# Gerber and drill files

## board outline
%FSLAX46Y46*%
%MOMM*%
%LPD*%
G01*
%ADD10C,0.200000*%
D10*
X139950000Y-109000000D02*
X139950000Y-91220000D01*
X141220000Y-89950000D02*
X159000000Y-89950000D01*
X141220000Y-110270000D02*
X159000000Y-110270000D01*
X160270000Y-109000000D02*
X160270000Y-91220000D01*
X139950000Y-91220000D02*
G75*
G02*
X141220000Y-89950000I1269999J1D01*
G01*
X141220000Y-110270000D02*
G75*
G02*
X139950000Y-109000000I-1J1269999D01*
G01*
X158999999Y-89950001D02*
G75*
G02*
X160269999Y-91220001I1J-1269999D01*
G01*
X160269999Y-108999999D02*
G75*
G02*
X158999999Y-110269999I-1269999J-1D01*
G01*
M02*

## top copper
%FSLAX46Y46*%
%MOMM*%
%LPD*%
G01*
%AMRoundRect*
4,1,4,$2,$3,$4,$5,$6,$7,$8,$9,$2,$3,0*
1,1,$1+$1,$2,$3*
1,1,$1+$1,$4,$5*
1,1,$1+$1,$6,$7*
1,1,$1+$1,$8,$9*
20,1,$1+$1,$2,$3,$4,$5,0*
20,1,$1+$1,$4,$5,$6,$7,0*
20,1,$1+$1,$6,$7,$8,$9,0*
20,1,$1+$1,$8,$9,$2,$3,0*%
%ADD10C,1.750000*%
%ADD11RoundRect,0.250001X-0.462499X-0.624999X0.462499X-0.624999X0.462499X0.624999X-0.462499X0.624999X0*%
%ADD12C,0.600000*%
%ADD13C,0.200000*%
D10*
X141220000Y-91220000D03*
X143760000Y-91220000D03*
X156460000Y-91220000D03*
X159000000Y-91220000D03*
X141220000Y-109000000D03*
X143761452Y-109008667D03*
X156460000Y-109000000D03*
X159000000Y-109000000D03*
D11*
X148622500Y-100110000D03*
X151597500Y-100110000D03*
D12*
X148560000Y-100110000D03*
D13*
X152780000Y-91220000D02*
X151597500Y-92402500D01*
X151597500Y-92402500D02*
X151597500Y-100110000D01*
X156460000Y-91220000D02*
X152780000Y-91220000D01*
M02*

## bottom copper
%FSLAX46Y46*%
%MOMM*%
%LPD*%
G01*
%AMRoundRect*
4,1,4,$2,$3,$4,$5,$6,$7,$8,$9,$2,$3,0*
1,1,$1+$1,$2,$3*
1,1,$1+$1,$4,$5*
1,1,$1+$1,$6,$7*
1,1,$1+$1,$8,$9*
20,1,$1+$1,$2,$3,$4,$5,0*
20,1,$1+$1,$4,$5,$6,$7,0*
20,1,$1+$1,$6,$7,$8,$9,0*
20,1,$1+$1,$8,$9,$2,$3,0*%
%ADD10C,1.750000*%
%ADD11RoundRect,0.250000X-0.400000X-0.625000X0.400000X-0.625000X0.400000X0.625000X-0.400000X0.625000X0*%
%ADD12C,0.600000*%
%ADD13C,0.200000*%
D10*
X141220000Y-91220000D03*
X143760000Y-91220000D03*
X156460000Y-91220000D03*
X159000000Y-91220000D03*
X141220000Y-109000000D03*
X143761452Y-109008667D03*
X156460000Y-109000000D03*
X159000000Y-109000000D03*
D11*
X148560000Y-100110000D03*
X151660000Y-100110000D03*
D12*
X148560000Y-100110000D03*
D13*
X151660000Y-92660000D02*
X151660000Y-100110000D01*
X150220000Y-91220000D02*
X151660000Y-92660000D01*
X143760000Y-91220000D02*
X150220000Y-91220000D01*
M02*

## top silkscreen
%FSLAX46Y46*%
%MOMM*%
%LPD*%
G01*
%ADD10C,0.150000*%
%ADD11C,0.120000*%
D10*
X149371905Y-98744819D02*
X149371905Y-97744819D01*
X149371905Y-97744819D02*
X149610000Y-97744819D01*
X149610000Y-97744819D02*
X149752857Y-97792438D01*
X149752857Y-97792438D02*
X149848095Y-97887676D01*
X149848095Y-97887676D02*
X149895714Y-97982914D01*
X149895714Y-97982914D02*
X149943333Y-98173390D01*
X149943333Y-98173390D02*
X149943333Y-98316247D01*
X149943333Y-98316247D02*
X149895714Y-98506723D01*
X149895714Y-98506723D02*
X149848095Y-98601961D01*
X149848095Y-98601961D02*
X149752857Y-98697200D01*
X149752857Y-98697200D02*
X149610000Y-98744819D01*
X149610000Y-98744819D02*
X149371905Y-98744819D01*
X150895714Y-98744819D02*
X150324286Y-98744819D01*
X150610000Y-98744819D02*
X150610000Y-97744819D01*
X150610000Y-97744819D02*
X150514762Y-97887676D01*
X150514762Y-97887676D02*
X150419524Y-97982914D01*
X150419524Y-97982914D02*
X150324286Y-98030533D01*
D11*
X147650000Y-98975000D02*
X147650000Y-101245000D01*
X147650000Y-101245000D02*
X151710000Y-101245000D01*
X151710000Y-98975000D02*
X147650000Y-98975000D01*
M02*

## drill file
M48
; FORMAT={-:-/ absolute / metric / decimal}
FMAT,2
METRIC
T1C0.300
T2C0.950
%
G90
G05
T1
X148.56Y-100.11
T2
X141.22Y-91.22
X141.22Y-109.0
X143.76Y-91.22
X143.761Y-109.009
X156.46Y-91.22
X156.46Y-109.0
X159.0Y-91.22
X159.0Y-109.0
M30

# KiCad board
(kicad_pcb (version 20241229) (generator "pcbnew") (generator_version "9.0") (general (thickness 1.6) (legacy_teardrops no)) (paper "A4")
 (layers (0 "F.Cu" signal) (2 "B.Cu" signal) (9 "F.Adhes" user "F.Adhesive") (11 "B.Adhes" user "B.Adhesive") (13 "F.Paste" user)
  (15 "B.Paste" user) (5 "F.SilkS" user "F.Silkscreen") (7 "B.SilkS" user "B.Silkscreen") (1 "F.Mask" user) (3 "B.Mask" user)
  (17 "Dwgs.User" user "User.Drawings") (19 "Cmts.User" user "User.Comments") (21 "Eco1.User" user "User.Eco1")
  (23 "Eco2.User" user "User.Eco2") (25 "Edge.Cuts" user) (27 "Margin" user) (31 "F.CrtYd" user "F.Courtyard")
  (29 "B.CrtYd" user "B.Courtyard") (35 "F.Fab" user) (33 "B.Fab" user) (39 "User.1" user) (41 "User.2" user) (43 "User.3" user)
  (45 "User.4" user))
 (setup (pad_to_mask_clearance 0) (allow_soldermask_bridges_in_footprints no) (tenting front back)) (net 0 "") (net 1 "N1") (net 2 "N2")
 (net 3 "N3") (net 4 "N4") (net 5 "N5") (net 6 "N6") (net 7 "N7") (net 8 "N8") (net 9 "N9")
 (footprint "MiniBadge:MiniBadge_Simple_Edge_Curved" (layer "F.Cu") (at 150.11 100.11)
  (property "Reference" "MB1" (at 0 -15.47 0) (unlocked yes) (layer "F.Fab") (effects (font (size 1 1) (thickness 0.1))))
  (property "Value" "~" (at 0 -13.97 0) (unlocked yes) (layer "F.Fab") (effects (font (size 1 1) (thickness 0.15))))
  (fp_line (start -10.16 8.89) (end -10.16 -8.89) (stroke (width 0.2) (type solid)) (layer "Edge.Cuts"))
  (fp_line (start -8.89 -10.16) (end 8.89 -10.16) (stroke (width 0.2) (type solid)) (layer "Edge.Cuts"))
  (fp_line (start -8.89 10.16) (end 8.89 10.16) (stroke (width 0.2) (type solid)) (layer "Edge.Cuts"))
  (fp_line (start 10.16 8.89) (end 10.16 -8.89) (stroke (width 0.2) (type solid)) (layer "Edge.Cuts"))
  (fp_arc (start -10.16 -8.89) (mid -9.788026 -9.788026) (end -8.89 -10.16) (stroke (width 0.2) (type solid)) (layer "Edge.Cuts"))
  (fp_arc (start -8.89 10.16) (mid -9.788026 9.788026) (end -10.16 8.89) (stroke (width 0.2) (type solid)) (layer "Edge.Cuts"))
  (fp_arc (start 8.889999 -10.159999) (mid 9.788025 -9.788025) (end 10.159999 -8.889999) (stroke (width 0.2) (type solid))
   (layer "Edge.Cuts"))
  (fp_arc (start 10.159999 8.889999) (mid 9.788025 9.788025) (end 8.889999 10.159999) (stroke (width 0.2) (type solid)) (layer "Edge.Cuts"))
  (pad "1" thru_hole circle (at -8.89 -8.89) (size 1.75 1.75) (drill 0.95) (layers "*.Cu" "*.Mask") (remove_unused_layers no) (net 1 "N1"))
  (pad "2" thru_hole circle (at -6.35 -8.89) (size 1.75 1.75) (drill 0.95) (layers "*.Cu" "*.Mask") (remove_unused_layers no) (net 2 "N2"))
  (pad "7" thru_hole circle (at 6.35 -8.89) (size 1.75 1.75) (drill 0.95) (layers "*.Cu" "*.Mask") (remove_unused_layers no) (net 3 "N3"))
  (pad "8" thru_hole circle (at 8.89 -8.89) (size 1.75 1.75) (drill 0.95) (layers "*.Cu" "*.Mask") (remove_unused_layers no) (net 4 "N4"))
  (pad "9" thru_hole circle (at -8.89 8.89) (size 1.75 1.75) (drill 0.95) (layers "*.Cu" "*.Mask") (remove_unused_layers no) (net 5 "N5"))
  (pad "10" thru_hole circle (at -6.348548 8.898667) (size 1.75 1.75) (drill 0.95) (layers "*.Cu" "*.Mask") (remove_unused_layers no)
   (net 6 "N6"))
  (pad "15" thru_hole circle (at 6.35 8.89) (size 1.75 1.75) (drill 0.95) (layers "*.Cu" "*.Mask") (remove_unused_layers no) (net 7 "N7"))
  (pad "16" thru_hole circle (at 8.89 8.89) (size 1.75 1.75) (drill 0.95) (layers "*.Cu" "*.Mask") (remove_unused_layers no) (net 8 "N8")))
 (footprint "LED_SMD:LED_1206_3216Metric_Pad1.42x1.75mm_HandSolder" (layer "F.Cu") (at 150.11 100.11)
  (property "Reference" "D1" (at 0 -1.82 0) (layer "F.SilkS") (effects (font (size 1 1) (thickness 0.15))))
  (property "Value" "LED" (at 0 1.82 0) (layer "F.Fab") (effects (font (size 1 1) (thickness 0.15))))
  (fp_line (start -2.46 -1.135) (end -2.46 1.135) (stroke (width 0.12) (type solid)) (layer "F.SilkS"))
  (fp_line (start -2.46 1.135) (end 1.6 1.135) (stroke (width 0.12) (type solid)) (layer "F.SilkS"))
  (fp_line (start 1.6 -1.135) (end -2.46 -1.135) (stroke (width 0.12) (type solid)) (layer "F.SilkS"))
  (pad "1" smd roundrect (at -1.4875 0) (size 1.425 1.75) (layers "F.Cu" "F.Mask" "F.Paste") (roundrect_rratio 0.175439) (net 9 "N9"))
  (pad "2" smd roundrect (at 1.4875 0) (size 1.425 1.75) (layers "F.Cu" "F.Mask" "F.Paste") (roundrect_rratio 0.175439) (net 3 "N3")))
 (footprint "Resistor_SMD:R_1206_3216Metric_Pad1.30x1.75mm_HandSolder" (layer "B.Cu") (at 150.11 100.11)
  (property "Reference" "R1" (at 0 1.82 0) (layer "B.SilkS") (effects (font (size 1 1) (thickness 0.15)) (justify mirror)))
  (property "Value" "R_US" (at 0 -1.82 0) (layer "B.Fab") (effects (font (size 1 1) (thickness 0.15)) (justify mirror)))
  (pad "1" smd roundrect (at -1.55 0) (size 1.3 1.75) (layers "B.Cu" "B.Mask" "B.Paste") (roundrect_rratio 0.192308) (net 9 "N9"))
  (pad "2" smd roundrect (at 1.55 0) (size 1.3 1.75) (layers "B.Cu" "B.Mask" "B.Paste") (roundrect_rratio 0.192308) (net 2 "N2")))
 (segment (start 152.78 91.22) (end 151.5975 92.4025) (width 0.2) (layer "F.Cu") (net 3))
 (segment (start 151.5975 92.4025) (end 151.5975 100.11) (width 0.2) (layer "F.Cu") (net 3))
 (segment (start 156.46 91.22) (end 152.78 91.22) (width 0.2) (layer "F.Cu") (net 3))
 (via (at 148.56 100.11) (size 0.6) (drill 0.3) (layers "F.Cu" "B.Cu") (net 9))
 (segment (start 151.66 92.66) (end 151.66 100.11) (width 0.2) (layer "B.Cu") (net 2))
 (segment (start 150.22 91.22) (end 151.66 92.66) (width 0.2) (layer "B.Cu") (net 2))
 (segment (start 143.76 91.22) (end 150.22 91.22) (width 0.2) (layer "B.Cu") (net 2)))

